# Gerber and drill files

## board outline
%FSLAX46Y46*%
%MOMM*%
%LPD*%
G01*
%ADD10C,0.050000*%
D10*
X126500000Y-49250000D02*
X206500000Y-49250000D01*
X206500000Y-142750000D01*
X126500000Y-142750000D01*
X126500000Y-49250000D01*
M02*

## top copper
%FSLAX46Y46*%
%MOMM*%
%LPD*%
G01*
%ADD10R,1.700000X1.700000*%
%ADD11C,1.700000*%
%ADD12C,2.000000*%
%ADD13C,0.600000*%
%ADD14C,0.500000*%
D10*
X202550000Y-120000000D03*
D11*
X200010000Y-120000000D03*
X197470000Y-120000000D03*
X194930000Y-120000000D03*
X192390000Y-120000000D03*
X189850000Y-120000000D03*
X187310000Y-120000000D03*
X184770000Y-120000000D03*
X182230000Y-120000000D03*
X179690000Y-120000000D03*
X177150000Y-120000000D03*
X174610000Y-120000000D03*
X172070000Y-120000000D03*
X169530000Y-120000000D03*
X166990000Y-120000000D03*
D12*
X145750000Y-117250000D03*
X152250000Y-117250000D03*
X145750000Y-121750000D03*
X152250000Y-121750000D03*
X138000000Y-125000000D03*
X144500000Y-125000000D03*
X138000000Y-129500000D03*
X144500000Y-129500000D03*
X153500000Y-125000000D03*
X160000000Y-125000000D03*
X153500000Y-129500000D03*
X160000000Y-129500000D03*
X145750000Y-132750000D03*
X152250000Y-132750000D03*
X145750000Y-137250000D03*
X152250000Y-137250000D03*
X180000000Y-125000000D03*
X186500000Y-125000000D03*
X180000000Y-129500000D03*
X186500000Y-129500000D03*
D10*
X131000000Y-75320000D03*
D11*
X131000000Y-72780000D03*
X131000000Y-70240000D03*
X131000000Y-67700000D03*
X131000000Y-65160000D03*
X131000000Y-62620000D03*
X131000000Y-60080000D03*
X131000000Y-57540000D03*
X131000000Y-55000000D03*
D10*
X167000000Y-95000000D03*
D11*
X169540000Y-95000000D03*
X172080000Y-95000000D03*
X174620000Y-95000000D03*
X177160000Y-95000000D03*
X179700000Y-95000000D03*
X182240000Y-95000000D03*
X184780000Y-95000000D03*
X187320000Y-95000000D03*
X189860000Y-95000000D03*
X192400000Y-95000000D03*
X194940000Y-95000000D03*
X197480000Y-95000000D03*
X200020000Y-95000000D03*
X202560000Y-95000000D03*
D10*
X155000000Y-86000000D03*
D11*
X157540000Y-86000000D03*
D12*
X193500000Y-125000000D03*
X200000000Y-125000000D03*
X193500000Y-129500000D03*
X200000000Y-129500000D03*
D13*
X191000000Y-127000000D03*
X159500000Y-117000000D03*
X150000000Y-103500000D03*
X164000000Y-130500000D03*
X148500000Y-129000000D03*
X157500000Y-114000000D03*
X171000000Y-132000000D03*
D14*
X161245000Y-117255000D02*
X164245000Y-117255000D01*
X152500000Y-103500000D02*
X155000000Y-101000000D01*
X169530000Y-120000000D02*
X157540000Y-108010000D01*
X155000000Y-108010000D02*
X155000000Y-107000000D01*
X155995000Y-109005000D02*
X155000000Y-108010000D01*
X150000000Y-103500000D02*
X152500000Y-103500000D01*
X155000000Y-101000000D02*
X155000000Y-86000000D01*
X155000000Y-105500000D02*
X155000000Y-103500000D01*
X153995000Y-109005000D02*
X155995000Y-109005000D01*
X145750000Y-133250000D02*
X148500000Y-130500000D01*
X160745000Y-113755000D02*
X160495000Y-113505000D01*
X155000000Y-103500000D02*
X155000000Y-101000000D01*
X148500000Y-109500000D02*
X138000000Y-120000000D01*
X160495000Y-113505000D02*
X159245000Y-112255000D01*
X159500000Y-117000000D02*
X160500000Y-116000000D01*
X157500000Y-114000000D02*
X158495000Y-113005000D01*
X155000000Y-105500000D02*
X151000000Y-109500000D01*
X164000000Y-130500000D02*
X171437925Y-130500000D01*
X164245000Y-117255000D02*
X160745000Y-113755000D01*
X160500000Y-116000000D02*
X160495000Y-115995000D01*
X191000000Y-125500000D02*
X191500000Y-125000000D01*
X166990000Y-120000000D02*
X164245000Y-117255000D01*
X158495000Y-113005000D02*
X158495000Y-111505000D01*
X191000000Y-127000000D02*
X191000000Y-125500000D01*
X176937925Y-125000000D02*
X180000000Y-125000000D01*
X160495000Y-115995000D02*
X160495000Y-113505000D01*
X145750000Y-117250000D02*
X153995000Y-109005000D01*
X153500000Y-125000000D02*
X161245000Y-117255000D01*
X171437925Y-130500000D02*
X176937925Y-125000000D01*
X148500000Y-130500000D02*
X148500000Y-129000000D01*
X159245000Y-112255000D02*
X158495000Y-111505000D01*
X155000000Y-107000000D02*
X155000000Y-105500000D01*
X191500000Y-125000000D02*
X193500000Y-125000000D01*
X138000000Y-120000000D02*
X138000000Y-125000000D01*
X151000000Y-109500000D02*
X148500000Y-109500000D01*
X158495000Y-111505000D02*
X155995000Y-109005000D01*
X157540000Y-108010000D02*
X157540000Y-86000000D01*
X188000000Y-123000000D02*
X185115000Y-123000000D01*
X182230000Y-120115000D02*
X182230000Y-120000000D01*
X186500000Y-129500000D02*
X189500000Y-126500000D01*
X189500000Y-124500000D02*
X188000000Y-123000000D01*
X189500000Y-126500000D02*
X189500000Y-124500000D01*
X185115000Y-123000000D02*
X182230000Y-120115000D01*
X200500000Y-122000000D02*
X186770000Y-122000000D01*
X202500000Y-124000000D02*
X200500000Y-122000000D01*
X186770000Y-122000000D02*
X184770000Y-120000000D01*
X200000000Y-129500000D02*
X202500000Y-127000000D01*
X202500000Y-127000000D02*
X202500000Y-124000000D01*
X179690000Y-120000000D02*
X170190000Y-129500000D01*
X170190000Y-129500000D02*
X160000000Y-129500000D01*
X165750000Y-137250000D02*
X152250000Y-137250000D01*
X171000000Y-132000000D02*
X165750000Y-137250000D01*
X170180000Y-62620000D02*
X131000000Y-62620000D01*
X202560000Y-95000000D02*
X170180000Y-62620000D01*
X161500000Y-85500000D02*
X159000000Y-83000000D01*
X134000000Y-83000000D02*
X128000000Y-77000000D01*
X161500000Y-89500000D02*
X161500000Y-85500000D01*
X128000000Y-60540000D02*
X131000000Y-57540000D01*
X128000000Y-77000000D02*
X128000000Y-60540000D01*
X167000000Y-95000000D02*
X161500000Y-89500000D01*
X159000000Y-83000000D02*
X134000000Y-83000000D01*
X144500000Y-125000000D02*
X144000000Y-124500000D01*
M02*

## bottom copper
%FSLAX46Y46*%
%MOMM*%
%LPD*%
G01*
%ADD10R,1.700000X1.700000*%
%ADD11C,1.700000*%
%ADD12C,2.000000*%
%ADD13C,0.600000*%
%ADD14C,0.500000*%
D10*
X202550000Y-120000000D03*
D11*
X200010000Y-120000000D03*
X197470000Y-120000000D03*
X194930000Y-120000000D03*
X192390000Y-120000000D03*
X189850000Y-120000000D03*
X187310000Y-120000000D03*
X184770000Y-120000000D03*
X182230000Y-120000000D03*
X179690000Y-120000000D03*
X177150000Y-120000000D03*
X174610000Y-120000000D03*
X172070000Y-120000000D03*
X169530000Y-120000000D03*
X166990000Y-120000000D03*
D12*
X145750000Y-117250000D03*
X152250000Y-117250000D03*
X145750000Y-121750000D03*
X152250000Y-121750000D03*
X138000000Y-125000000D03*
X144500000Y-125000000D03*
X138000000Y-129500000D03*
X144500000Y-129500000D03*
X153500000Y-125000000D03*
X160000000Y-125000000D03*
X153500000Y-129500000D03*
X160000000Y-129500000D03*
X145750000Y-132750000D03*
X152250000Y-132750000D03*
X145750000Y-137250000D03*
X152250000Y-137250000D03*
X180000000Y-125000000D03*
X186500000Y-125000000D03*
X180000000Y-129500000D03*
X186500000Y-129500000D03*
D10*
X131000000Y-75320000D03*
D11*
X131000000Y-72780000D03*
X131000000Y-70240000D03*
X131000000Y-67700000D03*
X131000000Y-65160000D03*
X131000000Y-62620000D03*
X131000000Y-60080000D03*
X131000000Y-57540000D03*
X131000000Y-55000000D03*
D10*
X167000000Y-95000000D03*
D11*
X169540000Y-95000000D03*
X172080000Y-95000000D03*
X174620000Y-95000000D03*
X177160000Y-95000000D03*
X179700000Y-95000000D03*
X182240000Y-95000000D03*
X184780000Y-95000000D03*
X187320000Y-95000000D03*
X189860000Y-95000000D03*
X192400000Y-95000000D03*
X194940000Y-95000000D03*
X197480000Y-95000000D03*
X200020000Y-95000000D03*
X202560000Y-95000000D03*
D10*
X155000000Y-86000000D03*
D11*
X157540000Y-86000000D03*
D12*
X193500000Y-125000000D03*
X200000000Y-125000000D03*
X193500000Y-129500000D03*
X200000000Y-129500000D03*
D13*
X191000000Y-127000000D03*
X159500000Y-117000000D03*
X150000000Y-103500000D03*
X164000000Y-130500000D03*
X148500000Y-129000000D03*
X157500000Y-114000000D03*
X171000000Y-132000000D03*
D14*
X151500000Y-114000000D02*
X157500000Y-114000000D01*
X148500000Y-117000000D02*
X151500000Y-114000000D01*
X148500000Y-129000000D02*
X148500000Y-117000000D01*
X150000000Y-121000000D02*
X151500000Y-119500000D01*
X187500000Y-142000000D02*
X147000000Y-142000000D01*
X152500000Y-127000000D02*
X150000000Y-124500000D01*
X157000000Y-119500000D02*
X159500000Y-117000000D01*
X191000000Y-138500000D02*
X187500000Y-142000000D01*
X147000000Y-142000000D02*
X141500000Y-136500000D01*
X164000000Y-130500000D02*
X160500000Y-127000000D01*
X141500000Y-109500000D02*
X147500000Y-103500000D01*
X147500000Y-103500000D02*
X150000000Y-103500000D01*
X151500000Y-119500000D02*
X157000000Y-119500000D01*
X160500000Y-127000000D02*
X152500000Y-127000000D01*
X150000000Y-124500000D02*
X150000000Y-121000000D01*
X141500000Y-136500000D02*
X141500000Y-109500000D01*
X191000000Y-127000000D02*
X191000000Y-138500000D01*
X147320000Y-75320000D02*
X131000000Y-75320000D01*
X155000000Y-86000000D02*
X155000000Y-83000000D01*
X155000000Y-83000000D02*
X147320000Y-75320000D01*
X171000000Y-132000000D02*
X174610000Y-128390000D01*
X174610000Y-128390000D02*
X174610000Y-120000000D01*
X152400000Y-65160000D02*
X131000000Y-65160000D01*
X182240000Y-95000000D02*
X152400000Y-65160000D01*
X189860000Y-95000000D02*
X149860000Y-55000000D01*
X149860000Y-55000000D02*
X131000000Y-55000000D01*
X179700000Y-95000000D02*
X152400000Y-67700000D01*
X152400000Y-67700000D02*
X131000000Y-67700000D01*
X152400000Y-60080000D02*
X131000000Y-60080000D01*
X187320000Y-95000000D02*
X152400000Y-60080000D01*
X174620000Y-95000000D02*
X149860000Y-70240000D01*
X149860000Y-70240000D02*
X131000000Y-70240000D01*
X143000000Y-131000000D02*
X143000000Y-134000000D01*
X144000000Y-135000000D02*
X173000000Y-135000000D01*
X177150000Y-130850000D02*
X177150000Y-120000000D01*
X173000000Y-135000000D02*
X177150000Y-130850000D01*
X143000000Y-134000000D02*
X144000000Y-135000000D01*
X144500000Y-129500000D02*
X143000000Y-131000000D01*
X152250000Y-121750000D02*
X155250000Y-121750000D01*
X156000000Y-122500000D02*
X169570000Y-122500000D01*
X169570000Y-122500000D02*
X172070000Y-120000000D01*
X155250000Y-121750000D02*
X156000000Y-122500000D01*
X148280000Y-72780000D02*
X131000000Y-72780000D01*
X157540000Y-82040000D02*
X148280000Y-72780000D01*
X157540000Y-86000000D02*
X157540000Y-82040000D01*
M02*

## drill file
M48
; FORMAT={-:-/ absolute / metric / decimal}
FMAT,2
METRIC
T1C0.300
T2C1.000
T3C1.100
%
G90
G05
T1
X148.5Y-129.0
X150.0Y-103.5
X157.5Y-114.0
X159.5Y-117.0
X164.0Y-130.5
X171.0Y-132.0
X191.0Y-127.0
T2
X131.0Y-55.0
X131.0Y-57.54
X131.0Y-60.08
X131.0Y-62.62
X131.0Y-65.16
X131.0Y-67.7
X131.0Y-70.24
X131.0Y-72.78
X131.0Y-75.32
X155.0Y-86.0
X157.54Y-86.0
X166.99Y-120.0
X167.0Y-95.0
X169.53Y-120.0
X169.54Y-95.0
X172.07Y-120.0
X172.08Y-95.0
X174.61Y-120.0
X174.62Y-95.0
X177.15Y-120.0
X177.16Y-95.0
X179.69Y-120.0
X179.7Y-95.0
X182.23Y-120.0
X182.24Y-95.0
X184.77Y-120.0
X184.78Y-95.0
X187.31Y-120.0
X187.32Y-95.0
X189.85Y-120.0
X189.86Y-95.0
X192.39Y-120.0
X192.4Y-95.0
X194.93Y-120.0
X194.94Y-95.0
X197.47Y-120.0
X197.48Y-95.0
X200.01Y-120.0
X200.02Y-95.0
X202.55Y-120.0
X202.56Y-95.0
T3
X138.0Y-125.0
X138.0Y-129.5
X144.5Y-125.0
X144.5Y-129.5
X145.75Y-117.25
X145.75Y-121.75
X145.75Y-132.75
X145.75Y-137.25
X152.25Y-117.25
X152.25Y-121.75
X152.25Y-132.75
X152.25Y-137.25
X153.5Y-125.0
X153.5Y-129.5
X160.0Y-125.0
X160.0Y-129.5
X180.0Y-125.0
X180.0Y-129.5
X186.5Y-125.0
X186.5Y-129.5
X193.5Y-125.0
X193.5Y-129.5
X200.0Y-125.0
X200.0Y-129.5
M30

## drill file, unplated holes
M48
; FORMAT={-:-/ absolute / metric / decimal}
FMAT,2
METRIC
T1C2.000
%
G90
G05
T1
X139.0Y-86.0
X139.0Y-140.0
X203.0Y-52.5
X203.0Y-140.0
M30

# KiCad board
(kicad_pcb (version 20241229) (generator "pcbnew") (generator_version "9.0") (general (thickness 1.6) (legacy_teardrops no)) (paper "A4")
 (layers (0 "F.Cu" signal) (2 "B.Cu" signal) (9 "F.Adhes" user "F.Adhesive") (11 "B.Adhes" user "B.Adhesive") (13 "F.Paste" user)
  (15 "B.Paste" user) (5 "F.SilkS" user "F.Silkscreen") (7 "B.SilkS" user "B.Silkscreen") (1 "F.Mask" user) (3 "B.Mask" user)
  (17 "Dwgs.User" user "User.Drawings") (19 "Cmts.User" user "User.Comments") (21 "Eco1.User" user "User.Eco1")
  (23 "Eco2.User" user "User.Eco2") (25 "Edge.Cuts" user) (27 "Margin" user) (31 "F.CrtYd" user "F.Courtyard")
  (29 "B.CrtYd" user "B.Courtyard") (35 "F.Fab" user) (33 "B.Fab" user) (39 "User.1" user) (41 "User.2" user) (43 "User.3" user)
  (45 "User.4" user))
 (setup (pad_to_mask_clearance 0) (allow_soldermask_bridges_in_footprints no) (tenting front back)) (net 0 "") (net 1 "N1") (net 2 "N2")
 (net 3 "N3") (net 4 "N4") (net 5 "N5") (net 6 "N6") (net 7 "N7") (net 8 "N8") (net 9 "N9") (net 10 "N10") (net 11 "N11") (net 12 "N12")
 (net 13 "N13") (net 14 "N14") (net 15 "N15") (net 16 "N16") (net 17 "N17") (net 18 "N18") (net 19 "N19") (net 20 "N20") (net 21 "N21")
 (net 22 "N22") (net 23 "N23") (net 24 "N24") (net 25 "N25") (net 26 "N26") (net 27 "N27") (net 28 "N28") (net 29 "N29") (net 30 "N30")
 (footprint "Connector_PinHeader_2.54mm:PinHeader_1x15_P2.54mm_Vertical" (layer "F.Cu") (at 202.55 120 -90)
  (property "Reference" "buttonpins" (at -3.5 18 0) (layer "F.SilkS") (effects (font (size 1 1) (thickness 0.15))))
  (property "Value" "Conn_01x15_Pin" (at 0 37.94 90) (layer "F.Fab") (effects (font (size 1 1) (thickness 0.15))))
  (pad "1" thru_hole rect (at 0 0 270) (size 1.7 1.7) (drill 1) (layers "*.Cu" "*.Mask") (remove_unused_layers no) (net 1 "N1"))
  (pad "2" thru_hole circle (at 0 2.54 270) (size 1.7 1.7) (drill 1) (layers "*.Cu" "*.Mask") (remove_unused_layers no) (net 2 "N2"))
  (pad "3" thru_hole circle (at 0 5.08 270) (size 1.7 1.7) (drill 1) (layers "*.Cu" "*.Mask") (remove_unused_layers no) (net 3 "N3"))
  (pad "4" thru_hole circle (at 0 7.62 270) (size 1.7 1.7) (drill 1) (layers "*.Cu" "*.Mask") (remove_unused_layers no) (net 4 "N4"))
  (pad "5" thru_hole circle (at 0 10.16 270) (size 1.7 1.7) (drill 1) (layers "*.Cu" "*.Mask") (remove_unused_layers no) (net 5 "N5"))
  (pad "6" thru_hole circle (at 0 12.7 270) (size 1.7 1.7) (drill 1) (layers "*.Cu" "*.Mask") (remove_unused_layers no) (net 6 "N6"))
  (pad "7" thru_hole circle (at 0 15.24 270) (size 1.7 1.7) (drill 1) (layers "*.Cu" "*.Mask") (remove_unused_layers no) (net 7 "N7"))
  (pad "8" thru_hole circle (at 0 17.78 270) (size 1.7 1.7) (drill 1) (layers "*.Cu" "*.Mask") (remove_unused_layers no) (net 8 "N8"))
  (pad "9" thru_hole circle (at 0 20.32 270) (size 1.7 1.7) (drill 1) (layers "*.Cu" "*.Mask") (remove_unused_layers no) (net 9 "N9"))
  (pad "10" thru_hole circle (at 0 22.86 270) (size 1.7 1.7) (drill 1) (layers "*.Cu" "*.Mask") (remove_unused_layers no) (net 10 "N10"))
  (pad "11" thru_hole circle (at 0 25.4 270) (size 1.7 1.7) (drill 1) (layers "*.Cu" "*.Mask") (remove_unused_layers no) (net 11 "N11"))
  (pad "12" thru_hole circle (at 0 27.94 270) (size 1.7 1.7) (drill 1) (layers "*.Cu" "*.Mask") (remove_unused_layers no) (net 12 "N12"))
  (pad "13" thru_hole circle (at 0 30.48 270) (size 1.7 1.7) (drill 1) (layers "*.Cu" "*.Mask") (remove_unused_layers no) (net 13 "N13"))
  (pad "14" thru_hole circle (at 0 33.02 270) (size 1.7 1.7) (drill 1) (layers "*.Cu" "*.Mask") (remove_unused_layers no) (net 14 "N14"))
  (pad "15" thru_hole circle (at 0 35.56 270) (size 1.7 1.7) (drill 1) (layers "*.Cu" "*.Mask") (remove_unused_layers no) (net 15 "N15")))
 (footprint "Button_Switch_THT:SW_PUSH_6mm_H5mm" (layer "F.Cu") (at 145.75 117.25)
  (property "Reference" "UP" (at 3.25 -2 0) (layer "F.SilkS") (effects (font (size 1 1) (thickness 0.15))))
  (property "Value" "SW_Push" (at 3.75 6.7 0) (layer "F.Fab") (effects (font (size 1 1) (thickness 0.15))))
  (pad "1" thru_hole circle (at 0 0 90) (size 2 2) (drill 1.1) (layers "*.Cu" "*.Mask") (remove_unused_layers no) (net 15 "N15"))
  (pad "1" thru_hole circle (at 6.5 0 90) (size 2 2) (drill 1.1) (layers "*.Cu" "*.Mask") (remove_unused_layers no) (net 15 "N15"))
  (pad "2" thru_hole circle (at 0 4.5 90) (size 2 2) (drill 1.1) (layers "*.Cu" "*.Mask") (remove_unused_layers no) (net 13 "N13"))
  (pad "2" thru_hole circle (at 6.5 4.5 90) (size 2 2) (drill 1.1) (layers "*.Cu" "*.Mask") (remove_unused_layers no) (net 13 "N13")))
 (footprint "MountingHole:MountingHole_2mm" (layer "F.Cu") (at 139 140)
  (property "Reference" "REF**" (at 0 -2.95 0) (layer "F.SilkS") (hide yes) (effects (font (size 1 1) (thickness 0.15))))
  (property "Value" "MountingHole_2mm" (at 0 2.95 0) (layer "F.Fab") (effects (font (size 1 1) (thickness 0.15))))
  (pad "" np_thru_hole circle (at 0 0) (size 2 2) (drill 2) (layers "*.Cu" "*.Mask")))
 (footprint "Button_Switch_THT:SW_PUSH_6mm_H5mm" (layer "F.Cu") (at 138 125)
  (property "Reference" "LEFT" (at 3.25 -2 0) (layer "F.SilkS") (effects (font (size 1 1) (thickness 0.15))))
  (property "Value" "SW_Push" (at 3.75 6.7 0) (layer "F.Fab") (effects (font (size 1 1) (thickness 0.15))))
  (pad "1" thru_hole circle (at 0 0 90) (size 2 2) (drill 1.1) (layers "*.Cu" "*.Mask") (remove_unused_layers no) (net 15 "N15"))
  (pad "1" thru_hole circle (at 6.5 0 90) (size 2 2) (drill 1.1) (layers "*.Cu" "*.Mask") (remove_unused_layers no) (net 15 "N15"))
  (pad "2" thru_hole circle (at 0 4.5 90) (size 2 2) (drill 1.1) (layers "*.Cu" "*.Mask") (remove_unused_layers no) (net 11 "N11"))
  (pad "2" thru_hole circle (at 6.5 4.5 90) (size 2 2) (drill 1.1) (layers "*.Cu" "*.Mask") (remove_unused_layers no) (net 11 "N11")))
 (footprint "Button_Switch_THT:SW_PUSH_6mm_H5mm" (layer "F.Cu") (at 153.5 125)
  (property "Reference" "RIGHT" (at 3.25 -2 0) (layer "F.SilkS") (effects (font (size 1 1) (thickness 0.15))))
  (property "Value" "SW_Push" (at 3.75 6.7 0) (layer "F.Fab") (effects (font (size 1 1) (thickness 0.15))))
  (pad "1" thru_hole circle (at 0 0 90) (size 2 2) (drill 1.1) (layers "*.Cu" "*.Mask") (remove_unused_layers no) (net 15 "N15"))
  (pad "1" thru_hole circle (at 6.5 0 90) (size 2 2) (drill 1.1) (layers "*.Cu" "*.Mask") (remove_unused_layers no) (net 15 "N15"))
  (pad "2" thru_hole circle (at 0 4.5 90) (size 2 2) (drill 1.1) (layers "*.Cu" "*.Mask") (remove_unused_layers no) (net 10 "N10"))
  (pad "2" thru_hole circle (at 6.5 4.5 90) (size 2 2) (drill 1.1) (layers "*.Cu" "*.Mask") (remove_unused_layers no) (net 10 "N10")))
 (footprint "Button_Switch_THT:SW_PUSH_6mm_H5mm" (layer "F.Cu") (at 145.75 132.75)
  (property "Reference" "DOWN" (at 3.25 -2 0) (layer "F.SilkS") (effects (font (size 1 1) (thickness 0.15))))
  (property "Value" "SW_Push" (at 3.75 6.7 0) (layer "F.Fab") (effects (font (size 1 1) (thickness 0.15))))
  (pad "1" thru_hole circle (at 0 0 90) (size 2 2) (drill 1.1) (layers "*.Cu" "*.Mask") (remove_unused_layers no) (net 15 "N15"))
  (pad "1" thru_hole circle (at 6.5 0 90) (size 2 2) (drill 1.1) (layers "*.Cu" "*.Mask") (remove_unused_layers no) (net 15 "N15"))
  (pad "2" thru_hole circle (at 0 4.5 90) (size 2 2) (drill 1.1) (layers "*.Cu" "*.Mask") (remove_unused_layers no) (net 12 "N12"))
  (pad "2" thru_hole circle (at 6.5 4.5 90) (size 2 2) (drill 1.1) (layers "*.Cu" "*.Mask") (remove_unused_layers no) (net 12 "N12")))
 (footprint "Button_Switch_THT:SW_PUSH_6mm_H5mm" (layer "F.Cu") (at 180 125)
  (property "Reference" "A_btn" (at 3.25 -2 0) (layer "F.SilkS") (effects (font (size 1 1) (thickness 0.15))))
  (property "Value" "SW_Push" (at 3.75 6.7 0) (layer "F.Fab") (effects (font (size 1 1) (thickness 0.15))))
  (pad "1" thru_hole circle (at 0 0 90) (size 2 2) (drill 1.1) (layers "*.Cu" "*.Mask") (remove_unused_layers no) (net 15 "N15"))
  (pad "1" thru_hole circle (at 6.5 0 90) (size 2 2) (drill 1.1) (layers "*.Cu" "*.Mask") (remove_unused_layers no) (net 15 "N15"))
  (pad "2" thru_hole circle (at 0 4.5 90) (size 2 2) (drill 1.1) (layers "*.Cu" "*.Mask") (remove_unused_layers no) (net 9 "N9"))
  (pad "2" thru_hole circle (at 6.5 4.5 90) (size 2 2) (drill 1.1) (layers "*.Cu" "*.Mask") (remove_unused_layers no) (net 9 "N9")))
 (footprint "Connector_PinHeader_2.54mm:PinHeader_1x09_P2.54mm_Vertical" (layer "F.Cu") (at 131 75.32 180)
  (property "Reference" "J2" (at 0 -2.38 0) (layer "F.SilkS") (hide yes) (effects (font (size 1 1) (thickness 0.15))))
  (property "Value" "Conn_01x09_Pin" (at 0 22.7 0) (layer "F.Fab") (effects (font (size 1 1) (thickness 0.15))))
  (pad "1" thru_hole rect (at 0 0 180) (size 1.7 1.7) (drill 1) (layers "*.Cu" "*.Mask") (remove_unused_layers no) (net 14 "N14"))
  (pad "2" thru_hole circle (at 0 2.54 180) (size 1.7 1.7) (drill 1) (layers "*.Cu" "*.Mask") (remove_unused_layers no) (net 15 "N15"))
  (pad "3" thru_hole circle (at 0 5.08 180) (size 1.7 1.7) (drill 1) (layers "*.Cu" "*.Mask") (remove_unused_layers no) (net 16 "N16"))
  (pad "4" thru_hole circle (at 0 7.62 180) (size 1.7 1.7) (drill 1) (layers "*.Cu" "*.Mask") (remove_unused_layers no) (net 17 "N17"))
  (pad "5" thru_hole circle (at 0 10.16 180) (size 1.7 1.7) (drill 1) (layers "*.Cu" "*.Mask") (remove_unused_layers no) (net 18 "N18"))
  (pad "6" thru_hole circle (at 0 12.7 180) (size 1.7 1.7) (drill 1) (layers "*.Cu" "*.Mask") (remove_unused_layers no) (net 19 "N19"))
  (pad "7" thru_hole circle (at 0 15.24 180) (size 1.7 1.7) (drill 1) (layers "*.Cu" "*.Mask") (remove_unused_layers no) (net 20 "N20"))
  (pad "8" thru_hole circle (at 0 17.78 180) (size 1.7 1.7) (drill 1) (layers "*.Cu" "*.Mask") (remove_unused_layers no) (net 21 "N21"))
  (pad "9" thru_hole circle (at 0 20.32 180) (size 1.7 1.7) (drill 1) (layers "*.Cu" "*.Mask") (remove_unused_layers no) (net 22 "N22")))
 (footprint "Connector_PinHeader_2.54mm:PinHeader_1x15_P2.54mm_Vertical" (layer "F.Cu") (at 167 95 90)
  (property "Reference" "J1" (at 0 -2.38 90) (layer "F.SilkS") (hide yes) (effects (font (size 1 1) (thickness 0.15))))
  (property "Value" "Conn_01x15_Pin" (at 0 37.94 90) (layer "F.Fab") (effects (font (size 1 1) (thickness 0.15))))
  (pad "1" thru_hole rect (at 0 0 90) (size 1.7 1.7) (drill 1) (layers "*.Cu" "*.Mask") (remove_unused_layers no) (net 21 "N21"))
  (pad "2" thru_hole circle (at 0 2.54 90) (size 1.7 1.7) (drill 1) (layers "*.Cu" "*.Mask") (remove_unused_layers no) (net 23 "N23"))
  (pad "3" thru_hole circle (at 0 5.08 90) (size 1.7 1.7) (drill 1) (layers "*.Cu" "*.Mask") (remove_unused_layers no) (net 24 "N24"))
  (pad "4" thru_hole circle (at 0 7.62 90) (size 1.7 1.7) (drill 1) (layers "*.Cu" "*.Mask") (remove_unused_layers no) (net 16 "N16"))
  (pad "5" thru_hole circle (at 0 10.16 90) (size 1.7 1.7) (drill 1) (layers "*.Cu" "*.Mask") (remove_unused_layers no) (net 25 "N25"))
  (pad "6" thru_hole circle (at 0 12.7 90) (size 1.7 1.7) (drill 1) (layers "*.Cu" "*.Mask") (remove_unused_layers no) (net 17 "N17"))
  (pad "7" thru_hole circle (at 0 15.24 90) (size 1.7 1.7) (drill 1) (layers "*.Cu" "*.Mask") (remove_unused_layers no) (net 18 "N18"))
  (pad "8" thru_hole circle (at 0 17.78 90) (size 1.7 1.7) (drill 1) (layers "*.Cu" "*.Mask") (remove_unused_layers no) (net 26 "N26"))
  (pad "9" thru_hole circle (at 0 20.32 90) (size 1.7 1.7) (drill 1) (layers "*.Cu" "*.Mask") (remove_unused_layers no) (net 20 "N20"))
  (pad "10" thru_hole circle (at 0 22.86 90) (size 1.7 1.7) (drill 1) (layers "*.Cu" "*.Mask") (remove_unused_layers no) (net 22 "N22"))
  (pad "11" thru_hole circle (at 0 25.4 90) (size 1.7 1.7) (drill 1) (layers "*.Cu" "*.Mask") (remove_unused_layers no) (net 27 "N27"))
  (pad "12" thru_hole circle (at 0 27.94 90) (size 1.7 1.7) (drill 1) (layers "*.Cu" "*.Mask") (remove_unused_layers no) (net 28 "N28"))
  (pad "13" thru_hole circle (at 0 30.48 90) (size 1.7 1.7) (drill 1) (layers "*.Cu" "*.Mask") (remove_unused_layers no) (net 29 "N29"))
  (pad "14" thru_hole circle (at 0 33.02 90) (size 1.7 1.7) (drill 1) (layers "*.Cu" "*.Mask") (remove_unused_layers no) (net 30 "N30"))
  (pad "15" thru_hole circle (at 0 35.56 90) (size 1.7 1.7) (drill 1) (layers "*.Cu" "*.Mask") (remove_unused_layers no) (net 19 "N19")))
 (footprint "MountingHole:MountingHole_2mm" (layer "F.Cu") (at 203 52.5)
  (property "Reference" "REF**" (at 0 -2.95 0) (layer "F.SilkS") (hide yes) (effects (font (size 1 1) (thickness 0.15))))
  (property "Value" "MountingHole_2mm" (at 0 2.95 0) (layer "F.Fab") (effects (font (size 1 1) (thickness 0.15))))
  (pad "" np_thru_hole circle (at 0 0) (size 2 2) (drill 2) (layers "*.Cu" "*.Mask")))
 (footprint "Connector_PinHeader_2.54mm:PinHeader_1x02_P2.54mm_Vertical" (layer "F.Cu") (at 155 86 90)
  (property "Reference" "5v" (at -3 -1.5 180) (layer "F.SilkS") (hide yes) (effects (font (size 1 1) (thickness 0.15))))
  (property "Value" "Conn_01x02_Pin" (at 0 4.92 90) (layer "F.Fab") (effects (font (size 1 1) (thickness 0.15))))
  (pad "1" thru_hole rect (at 0 0 90) (size 1.7 1.7) (drill 1) (layers "*.Cu" "*.Mask") (remove_unused_layers no) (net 14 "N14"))
  (pad "2" thru_hole circle (at 0 2.54 90) (size 1.7 1.7) (drill 1) (layers "*.Cu" "*.Mask") (remove_unused_layers no) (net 15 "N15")))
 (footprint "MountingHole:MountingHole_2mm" (layer "F.Cu") (at 139 86)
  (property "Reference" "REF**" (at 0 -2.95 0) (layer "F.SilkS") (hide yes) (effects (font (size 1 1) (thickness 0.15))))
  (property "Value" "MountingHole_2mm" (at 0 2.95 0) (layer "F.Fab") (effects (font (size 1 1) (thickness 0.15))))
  (pad "" np_thru_hole circle (at 0 0) (size 2 2) (drill 2) (layers "*.Cu" "*.Mask")))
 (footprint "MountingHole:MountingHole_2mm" (layer "F.Cu") (at 203 140)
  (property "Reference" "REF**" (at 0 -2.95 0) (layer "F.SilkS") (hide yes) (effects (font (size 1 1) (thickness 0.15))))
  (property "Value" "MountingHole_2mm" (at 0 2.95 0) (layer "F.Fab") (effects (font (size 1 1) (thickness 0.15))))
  (pad "" np_thru_hole circle (at 0 0) (size 2 2) (drill 2) (layers "*.Cu" "*.Mask")))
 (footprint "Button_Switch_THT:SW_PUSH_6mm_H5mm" (layer "F.Cu") (at 193.5 125)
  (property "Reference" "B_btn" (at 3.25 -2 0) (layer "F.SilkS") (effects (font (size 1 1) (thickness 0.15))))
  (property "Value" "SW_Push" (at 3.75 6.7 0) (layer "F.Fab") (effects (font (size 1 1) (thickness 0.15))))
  (pad "1" thru_hole circle (at 0 0 90) (size 2 2) (drill 1.1) (layers "*.Cu" "*.Mask") (remove_unused_layers no) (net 15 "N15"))
  (pad "1" thru_hole circle (at 6.5 0 90) (size 2 2) (drill 1.1) (layers "*.Cu" "*.Mask") (remove_unused_layers no) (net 15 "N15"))
  (pad "2" thru_hole circle (at 0 4.5 90) (size 2 2) (drill 1.1) (layers "*.Cu" "*.Mask") (remove_unused_layers no) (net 8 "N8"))
  (pad "2" thru_hole circle (at 6.5 4.5 90) (size 2 2) (drill 1.1) (layers "*.Cu" "*.Mask") (remove_unused_layers no) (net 8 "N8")))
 (gr_rect (start 126.5 49.25) (end 206.5 142.75) (stroke (width 0.05) (type solid)) (fill no) (layer "Edge.Cuts"))
 (segment (start 161.245 117.255) (end 164.245 117.255) (width 0.5) (layer "F.Cu") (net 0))
 (segment (start 152.5 103.5) (end 155 101) (width 0.5) (layer "F.Cu") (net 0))
 (segment (start 169.53 120) (end 157.54 108.01) (width 0.5) (layer "F.Cu") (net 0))
 (segment (start 155 108.01) (end 155 107) (width 0.5) (layer "F.Cu") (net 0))
 (segment (start 155.995 109.005) (end 155 108.01) (width 0.5) (layer "F.Cu") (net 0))
 (segment (start 150 103.5) (end 152.5 103.5) (width 0.5) (layer "F.Cu") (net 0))
 (segment (start 155 101) (end 155 86) (width 0.5) (layer "F.Cu") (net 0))
 (segment (start 155 105.5) (end 155 103.5) (width 0.5) (layer "F.Cu") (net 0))
 (segment (start 153.995 109.005) (end 155.995 109.005) (width 0.5) (layer "F.Cu") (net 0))
 (segment (start 145.75 133.25) (end 148.5 130.5) (width 0.5) (layer "F.Cu") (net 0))
 (segment (start 160.745 113.755) (end 160.495 113.505) (width 0.5) (layer "F.Cu") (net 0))
 (segment (start 155 103.5) (end 155 101) (width 0.5) (layer "F.Cu") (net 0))
 (segment (start 148.5 109.5) (end 138 120) (width 0.5) (layer "F.Cu") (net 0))
 (segment (start 160.495 113.505) (end 159.245 112.255) (width 0.5) (layer "F.Cu") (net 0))
 (segment (start 159.5 117) (end 160.5 116) (width 0.5) (layer "F.Cu") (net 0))
 (segment (start 157.5 114) (end 158.495 113.005) (width 0.5) (layer "F.Cu") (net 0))
 (segment (start 155 105.5) (end 151 109.5) (width 0.5) (layer "F.Cu") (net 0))
 (segment (start 164 130.5) (end 171.437925 130.5) (width 0.5) (layer "F.Cu") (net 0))
 (segment (start 164.245 117.255) (end 160.745 113.755) (width 0.5) (layer "F.Cu") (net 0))
 (segment (start 160.5 116) (end 160.495 115.995) (width 0.5) (layer "F.Cu") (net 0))
 (segment (start 191 125.5) (end 191.5 125) (width 0.5) (layer "F.Cu") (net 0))
 (segment (start 166.99 120) (end 164.245 117.255) (width 0.5) (layer "F.Cu") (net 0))
 (segment (start 158.495 113.005) (end 158.495 111.505) (width 0.5) (layer "F.Cu") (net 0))
 (segment (start 191 127) (end 191 125.5) (width 0.5) (layer "F.Cu") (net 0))
 (segment (start 176.937925 125) (end 180 125) (width 0.5) (layer "F.Cu") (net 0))
 (segment (start 160.495 115.995) (end 160.495 113.505) (width 0.5) (layer "F.Cu") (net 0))
 (segment (start 145.75 117.25) (end 153.995 109.005) (width 0.5) (layer "F.Cu") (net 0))
 (segment (start 153.5 125) (end 161.245 117.255) (width 0.5) (layer "F.Cu") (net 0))
 (segment (start 171.437925 130.5) (end 176.937925 125) (width 0.5) (layer "F.Cu") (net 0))
 (segment (start 148.5 130.5) (end 148.5 129) (width 0.5) (layer "F.Cu") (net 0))
 (segment (start 159.245 112.255) (end 158.495 111.505) (width 0.5) (layer "F.Cu") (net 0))
 (segment (start 155 107) (end 155 105.5) (width 0.5) (layer "F.Cu") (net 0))
 (segment (start 191.5 125) (end 193.5 125) (width 0.5) (layer "F.Cu") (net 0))
 (segment (start 138 120) (end 138 125) (width 0.5) (layer "F.Cu") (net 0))
 (segment (start 151 109.5) (end 148.5 109.5) (width 0.5) (layer "F.Cu") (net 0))
 (segment (start 158.495 111.505) (end 155.995 109.005) (width 0.5) (layer "F.Cu") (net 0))
 (segment (start 157.54 108.01) (end 157.54 86) (width 0.5) (layer "F.Cu") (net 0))
 (via (at 191 127) (size 0.6) (drill 0.3) (layers "F.Cu" "B.Cu") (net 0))
 (via (at 159.5 117) (size 0.6) (drill 0.3) (layers "F.Cu" "B.Cu") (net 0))
 (via (at 150 103.5) (size 0.6) (drill 0.3) (layers "F.Cu" "B.Cu") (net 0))
 (via (at 164 130.5) (size 0.6) (drill 0.3) (layers "F.Cu" "B.Cu") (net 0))
 (via (at 148.5 129) (size 0.6) (drill 0.3) (layers "F.Cu" "B.Cu") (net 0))
 (via (at 157.5 114) (size 0.6) (drill 0.3) (layers "F.Cu" "B.Cu") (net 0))
 (segment (start 148.5 117) (end 151.5 114) (width 0.5) (layer "B.Cu") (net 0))
 (segment (start 148.5 129) (end 148.5 117) (width 0.5) (layer "B.Cu") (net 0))
 (segment (start 150 121) (end 151.5 119.5) (width 0.5) (layer "B.Cu") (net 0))
 (segment (start 187.5 142) (end 147 142) (width 0.5) (layer "B.Cu") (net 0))
 (segment (start 152.5 127) (end 150 124.5) (width 0.5) (layer "B.Cu") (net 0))
 (segment (start 157 119.5) (end 159.5 117) (width 0.5) (layer "B.Cu") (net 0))
 (segment (start 151.5 114) (end 157.5 114) (width 0.5) (layer "B.Cu") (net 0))
 (segment (start 191 138.5) (end 187.5 142) (width 0.5) (layer "B.Cu") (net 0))
 (segment (start 147 142) (end 141.5 136.5) (width 0.5) (layer "B.Cu") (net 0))
 (segment (start 164 130.5) (end 160.5 127) (width 0.5) (layer "B.Cu") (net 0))
 (segment (start 141.5 109.5) (end 147.5 103.5) (width 0.5) (layer "B.Cu") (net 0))
 (segment (start 147.5 103.5) (end 150 103.5) (width 0.5) (layer "B.Cu") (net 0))
 (segment (start 151.5 119.5) (end 157 119.5) (width 0.5) (layer "B.Cu") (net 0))
 (segment (start 160.5 127) (end 152.5 127) (width 0.5) (layer "B.Cu") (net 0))
 (segment (start 150 124.5) (end 150 121) (width 0.5) (layer "B.Cu") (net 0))
 (segment (start 141.5 136.5) (end 141.5 109.5) (width 0.5) (layer "B.Cu") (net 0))
 (segment (start 191 127) (end 191 138.5) (width 0.5) (layer "B.Cu") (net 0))
 (segment (start 188 123) (end 185.115 123) (width 0.5) (layer "F.Cu") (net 9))
 (segment (start 182.23 120.115) (end 182.23 120) (width 0.5) (layer "F.Cu") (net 9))
 (segment (start 186.5 129.5) (end 189.5 126.5) (width 0.5) (layer "F.Cu") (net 9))
 (segment (start 189.5 124.5) (end 188 123) (width 0.5) (layer "F.Cu") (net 9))
 (segment (start 189.5 126.5) (end 189.5 124.5) (width 0.5) (layer "F.Cu") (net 9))
 (segment (start 185.115 123) (end 182.23 120.115) (width 0.5) (layer "F.Cu") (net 9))
 (segment (start 147.32 75.32) (end 131 75.32) (width 0.5) (layer "B.Cu") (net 14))
 (segment (start 155 86) (end 155 83) (width 0.5) (layer "B.Cu") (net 14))
 (segment (start 155 83) (end 147.32 75.32) (width 0.5) (layer "B.Cu") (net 14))
 (segment (start 200.5 122) (end 186.77 122) (width 0.5) (layer "F.Cu") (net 8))
 (segment (start 202.5 124) (end 200.5 122) (width 0.5) (layer "F.Cu") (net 8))
 (segment (start 186.77 122) (end 184.77 120) (width 0.5) (layer "F.Cu") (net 8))
 (segment (start 200 129.5) (end 202.5 127) (width 0.5) (layer "F.Cu") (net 8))
 (segment (start 202.5 127) (end 202.5 124) (width 0.5) (layer "F.Cu") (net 8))
 (segment (start 179.69 120) (end 170.19 129.5) (width 0.5) (layer "F.Cu") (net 10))
 (segment (start 170.19 129.5) (end 160 129.5) (width 0.5) (layer "F.Cu") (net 10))
 (segment (start 165.75 137.25) (end 152.25 137.25) (width 0.5) (layer "F.Cu") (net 12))
 (segment (start 171 132) (end 165.75 137.25) (width 0.5) (layer "F.Cu") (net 12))
 (via (at 171 132) (size 0.6) (drill 0.3) (layers "F.Cu" "B.Cu") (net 12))
 (segment (start 171 132) (end 174.61 128.39) (width 0.5) (layer "B.Cu") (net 12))
 (segment (start 174.61 128.39) (end 174.61 120) (width 0.5) (layer "B.Cu") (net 12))
 (segment (start 152.4 65.16) (end 131 65.16) (width 0.5) (layer "B.Cu") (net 18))
 (segment (start 182.24 95) (end 152.4 65.16) (width 0.5) (layer "B.Cu") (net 18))
 (segment (start 189.86 95) (end 149.86 55) (width 0.5) (layer "B.Cu") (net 22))
 (segment (start 149.86 55) (end 131 55) (width 0.5) (layer "B.Cu") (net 22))
 (segment (start 170.18 62.62) (end 131 62.62) (width 0.5) (layer "F.Cu") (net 19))
 (segment (start 202.56 95) (end 170.18 62.62) (width 0.5) (layer "F.Cu") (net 19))
 (segment (start 179.7 95) (end 152.4 67.7) (width 0.5) (layer "B.Cu") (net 17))
 (segment (start 152.4 67.7) (end 131 67.7) (width 0.5) (layer "B.Cu") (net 17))
 (segment (start 152.4 60.08) (end 131 60.08) (width 0.5) (layer "B.Cu") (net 20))
 (segment (start 187.32 95) (end 152.4 60.08) (width 0.5) (layer "B.Cu") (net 20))
 (segment (start 161.5 85.5) (end 159 83) (width 0.5) (layer "F.Cu") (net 21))
 (segment (start 134 83) (end 128 77) (width 0.5) (layer "F.Cu") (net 21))
 (segment (start 161.5 89.5) (end 161.5 85.5) (width 0.5) (layer "F.Cu") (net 21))
 (segment (start 128 60.54) (end 131 57.54) (width 0.5) (layer "F.Cu") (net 21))
 (segment (start 128 77) (end 128 60.54) (width 0.5) (layer "F.Cu") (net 21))
 (segment (start 167 95) (end 161.5 89.5) (width 0.5) (layer "F.Cu") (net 21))
 (segment (start 159 83) (end 134 83) (width 0.5) (layer "F.Cu") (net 21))
 (segment (start 174.62 95) (end 149.86 70.24) (width 0.5) (layer "B.Cu") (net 16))
 (segment (start 149.86 70.24) (end 131 70.24) (width 0.5) (layer "B.Cu") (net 16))
 (segment (start 143 131) (end 143 134) (width 0.5) (layer "B.Cu") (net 11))
 (segment (start 144 135) (end 173 135) (width 0.5) (layer "B.Cu") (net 11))
 (segment (start 177.15 130.85) (end 177.15 120) (width 0.5) (layer "B.Cu") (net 11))
 (segment (start 173 135) (end 177.15 130.85) (width 0.5) (layer "B.Cu") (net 11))
 (segment (start 143 134) (end 144 135) (width 0.5) (layer "B.Cu") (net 11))
 (segment (start 144.5 129.5) (end 143 131) (width 0.5) (layer "B.Cu") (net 11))
 (segment (start 152.25 121.75) (end 155.25 121.75) (width 0.5) (layer "B.Cu") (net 13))
 (segment (start 156 122.5) (end 169.57 122.5) (width 0.5) (layer "B.Cu") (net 13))
 (segment (start 169.57 122.5) (end 172.07 120) (width 0.5) (layer "B.Cu") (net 13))
 (segment (start 155.25 121.75) (end 156 122.5) (width 0.5) (layer "B.Cu") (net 13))
 (segment (start 144.5 125) (end 144 124.5) (width 0.5) (layer "F.Cu") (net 15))
 (segment (start 148.28 72.78) (end 131 72.78) (width 0.5) (layer "B.Cu") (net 15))
 (segment (start 157.54 82.04) (end 148.28 72.78) (width 0.5) (layer "B.Cu") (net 15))
 (segment (start 157.54 86) (end 157.54 82.04) (width 0.5) (layer "B.Cu") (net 15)))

